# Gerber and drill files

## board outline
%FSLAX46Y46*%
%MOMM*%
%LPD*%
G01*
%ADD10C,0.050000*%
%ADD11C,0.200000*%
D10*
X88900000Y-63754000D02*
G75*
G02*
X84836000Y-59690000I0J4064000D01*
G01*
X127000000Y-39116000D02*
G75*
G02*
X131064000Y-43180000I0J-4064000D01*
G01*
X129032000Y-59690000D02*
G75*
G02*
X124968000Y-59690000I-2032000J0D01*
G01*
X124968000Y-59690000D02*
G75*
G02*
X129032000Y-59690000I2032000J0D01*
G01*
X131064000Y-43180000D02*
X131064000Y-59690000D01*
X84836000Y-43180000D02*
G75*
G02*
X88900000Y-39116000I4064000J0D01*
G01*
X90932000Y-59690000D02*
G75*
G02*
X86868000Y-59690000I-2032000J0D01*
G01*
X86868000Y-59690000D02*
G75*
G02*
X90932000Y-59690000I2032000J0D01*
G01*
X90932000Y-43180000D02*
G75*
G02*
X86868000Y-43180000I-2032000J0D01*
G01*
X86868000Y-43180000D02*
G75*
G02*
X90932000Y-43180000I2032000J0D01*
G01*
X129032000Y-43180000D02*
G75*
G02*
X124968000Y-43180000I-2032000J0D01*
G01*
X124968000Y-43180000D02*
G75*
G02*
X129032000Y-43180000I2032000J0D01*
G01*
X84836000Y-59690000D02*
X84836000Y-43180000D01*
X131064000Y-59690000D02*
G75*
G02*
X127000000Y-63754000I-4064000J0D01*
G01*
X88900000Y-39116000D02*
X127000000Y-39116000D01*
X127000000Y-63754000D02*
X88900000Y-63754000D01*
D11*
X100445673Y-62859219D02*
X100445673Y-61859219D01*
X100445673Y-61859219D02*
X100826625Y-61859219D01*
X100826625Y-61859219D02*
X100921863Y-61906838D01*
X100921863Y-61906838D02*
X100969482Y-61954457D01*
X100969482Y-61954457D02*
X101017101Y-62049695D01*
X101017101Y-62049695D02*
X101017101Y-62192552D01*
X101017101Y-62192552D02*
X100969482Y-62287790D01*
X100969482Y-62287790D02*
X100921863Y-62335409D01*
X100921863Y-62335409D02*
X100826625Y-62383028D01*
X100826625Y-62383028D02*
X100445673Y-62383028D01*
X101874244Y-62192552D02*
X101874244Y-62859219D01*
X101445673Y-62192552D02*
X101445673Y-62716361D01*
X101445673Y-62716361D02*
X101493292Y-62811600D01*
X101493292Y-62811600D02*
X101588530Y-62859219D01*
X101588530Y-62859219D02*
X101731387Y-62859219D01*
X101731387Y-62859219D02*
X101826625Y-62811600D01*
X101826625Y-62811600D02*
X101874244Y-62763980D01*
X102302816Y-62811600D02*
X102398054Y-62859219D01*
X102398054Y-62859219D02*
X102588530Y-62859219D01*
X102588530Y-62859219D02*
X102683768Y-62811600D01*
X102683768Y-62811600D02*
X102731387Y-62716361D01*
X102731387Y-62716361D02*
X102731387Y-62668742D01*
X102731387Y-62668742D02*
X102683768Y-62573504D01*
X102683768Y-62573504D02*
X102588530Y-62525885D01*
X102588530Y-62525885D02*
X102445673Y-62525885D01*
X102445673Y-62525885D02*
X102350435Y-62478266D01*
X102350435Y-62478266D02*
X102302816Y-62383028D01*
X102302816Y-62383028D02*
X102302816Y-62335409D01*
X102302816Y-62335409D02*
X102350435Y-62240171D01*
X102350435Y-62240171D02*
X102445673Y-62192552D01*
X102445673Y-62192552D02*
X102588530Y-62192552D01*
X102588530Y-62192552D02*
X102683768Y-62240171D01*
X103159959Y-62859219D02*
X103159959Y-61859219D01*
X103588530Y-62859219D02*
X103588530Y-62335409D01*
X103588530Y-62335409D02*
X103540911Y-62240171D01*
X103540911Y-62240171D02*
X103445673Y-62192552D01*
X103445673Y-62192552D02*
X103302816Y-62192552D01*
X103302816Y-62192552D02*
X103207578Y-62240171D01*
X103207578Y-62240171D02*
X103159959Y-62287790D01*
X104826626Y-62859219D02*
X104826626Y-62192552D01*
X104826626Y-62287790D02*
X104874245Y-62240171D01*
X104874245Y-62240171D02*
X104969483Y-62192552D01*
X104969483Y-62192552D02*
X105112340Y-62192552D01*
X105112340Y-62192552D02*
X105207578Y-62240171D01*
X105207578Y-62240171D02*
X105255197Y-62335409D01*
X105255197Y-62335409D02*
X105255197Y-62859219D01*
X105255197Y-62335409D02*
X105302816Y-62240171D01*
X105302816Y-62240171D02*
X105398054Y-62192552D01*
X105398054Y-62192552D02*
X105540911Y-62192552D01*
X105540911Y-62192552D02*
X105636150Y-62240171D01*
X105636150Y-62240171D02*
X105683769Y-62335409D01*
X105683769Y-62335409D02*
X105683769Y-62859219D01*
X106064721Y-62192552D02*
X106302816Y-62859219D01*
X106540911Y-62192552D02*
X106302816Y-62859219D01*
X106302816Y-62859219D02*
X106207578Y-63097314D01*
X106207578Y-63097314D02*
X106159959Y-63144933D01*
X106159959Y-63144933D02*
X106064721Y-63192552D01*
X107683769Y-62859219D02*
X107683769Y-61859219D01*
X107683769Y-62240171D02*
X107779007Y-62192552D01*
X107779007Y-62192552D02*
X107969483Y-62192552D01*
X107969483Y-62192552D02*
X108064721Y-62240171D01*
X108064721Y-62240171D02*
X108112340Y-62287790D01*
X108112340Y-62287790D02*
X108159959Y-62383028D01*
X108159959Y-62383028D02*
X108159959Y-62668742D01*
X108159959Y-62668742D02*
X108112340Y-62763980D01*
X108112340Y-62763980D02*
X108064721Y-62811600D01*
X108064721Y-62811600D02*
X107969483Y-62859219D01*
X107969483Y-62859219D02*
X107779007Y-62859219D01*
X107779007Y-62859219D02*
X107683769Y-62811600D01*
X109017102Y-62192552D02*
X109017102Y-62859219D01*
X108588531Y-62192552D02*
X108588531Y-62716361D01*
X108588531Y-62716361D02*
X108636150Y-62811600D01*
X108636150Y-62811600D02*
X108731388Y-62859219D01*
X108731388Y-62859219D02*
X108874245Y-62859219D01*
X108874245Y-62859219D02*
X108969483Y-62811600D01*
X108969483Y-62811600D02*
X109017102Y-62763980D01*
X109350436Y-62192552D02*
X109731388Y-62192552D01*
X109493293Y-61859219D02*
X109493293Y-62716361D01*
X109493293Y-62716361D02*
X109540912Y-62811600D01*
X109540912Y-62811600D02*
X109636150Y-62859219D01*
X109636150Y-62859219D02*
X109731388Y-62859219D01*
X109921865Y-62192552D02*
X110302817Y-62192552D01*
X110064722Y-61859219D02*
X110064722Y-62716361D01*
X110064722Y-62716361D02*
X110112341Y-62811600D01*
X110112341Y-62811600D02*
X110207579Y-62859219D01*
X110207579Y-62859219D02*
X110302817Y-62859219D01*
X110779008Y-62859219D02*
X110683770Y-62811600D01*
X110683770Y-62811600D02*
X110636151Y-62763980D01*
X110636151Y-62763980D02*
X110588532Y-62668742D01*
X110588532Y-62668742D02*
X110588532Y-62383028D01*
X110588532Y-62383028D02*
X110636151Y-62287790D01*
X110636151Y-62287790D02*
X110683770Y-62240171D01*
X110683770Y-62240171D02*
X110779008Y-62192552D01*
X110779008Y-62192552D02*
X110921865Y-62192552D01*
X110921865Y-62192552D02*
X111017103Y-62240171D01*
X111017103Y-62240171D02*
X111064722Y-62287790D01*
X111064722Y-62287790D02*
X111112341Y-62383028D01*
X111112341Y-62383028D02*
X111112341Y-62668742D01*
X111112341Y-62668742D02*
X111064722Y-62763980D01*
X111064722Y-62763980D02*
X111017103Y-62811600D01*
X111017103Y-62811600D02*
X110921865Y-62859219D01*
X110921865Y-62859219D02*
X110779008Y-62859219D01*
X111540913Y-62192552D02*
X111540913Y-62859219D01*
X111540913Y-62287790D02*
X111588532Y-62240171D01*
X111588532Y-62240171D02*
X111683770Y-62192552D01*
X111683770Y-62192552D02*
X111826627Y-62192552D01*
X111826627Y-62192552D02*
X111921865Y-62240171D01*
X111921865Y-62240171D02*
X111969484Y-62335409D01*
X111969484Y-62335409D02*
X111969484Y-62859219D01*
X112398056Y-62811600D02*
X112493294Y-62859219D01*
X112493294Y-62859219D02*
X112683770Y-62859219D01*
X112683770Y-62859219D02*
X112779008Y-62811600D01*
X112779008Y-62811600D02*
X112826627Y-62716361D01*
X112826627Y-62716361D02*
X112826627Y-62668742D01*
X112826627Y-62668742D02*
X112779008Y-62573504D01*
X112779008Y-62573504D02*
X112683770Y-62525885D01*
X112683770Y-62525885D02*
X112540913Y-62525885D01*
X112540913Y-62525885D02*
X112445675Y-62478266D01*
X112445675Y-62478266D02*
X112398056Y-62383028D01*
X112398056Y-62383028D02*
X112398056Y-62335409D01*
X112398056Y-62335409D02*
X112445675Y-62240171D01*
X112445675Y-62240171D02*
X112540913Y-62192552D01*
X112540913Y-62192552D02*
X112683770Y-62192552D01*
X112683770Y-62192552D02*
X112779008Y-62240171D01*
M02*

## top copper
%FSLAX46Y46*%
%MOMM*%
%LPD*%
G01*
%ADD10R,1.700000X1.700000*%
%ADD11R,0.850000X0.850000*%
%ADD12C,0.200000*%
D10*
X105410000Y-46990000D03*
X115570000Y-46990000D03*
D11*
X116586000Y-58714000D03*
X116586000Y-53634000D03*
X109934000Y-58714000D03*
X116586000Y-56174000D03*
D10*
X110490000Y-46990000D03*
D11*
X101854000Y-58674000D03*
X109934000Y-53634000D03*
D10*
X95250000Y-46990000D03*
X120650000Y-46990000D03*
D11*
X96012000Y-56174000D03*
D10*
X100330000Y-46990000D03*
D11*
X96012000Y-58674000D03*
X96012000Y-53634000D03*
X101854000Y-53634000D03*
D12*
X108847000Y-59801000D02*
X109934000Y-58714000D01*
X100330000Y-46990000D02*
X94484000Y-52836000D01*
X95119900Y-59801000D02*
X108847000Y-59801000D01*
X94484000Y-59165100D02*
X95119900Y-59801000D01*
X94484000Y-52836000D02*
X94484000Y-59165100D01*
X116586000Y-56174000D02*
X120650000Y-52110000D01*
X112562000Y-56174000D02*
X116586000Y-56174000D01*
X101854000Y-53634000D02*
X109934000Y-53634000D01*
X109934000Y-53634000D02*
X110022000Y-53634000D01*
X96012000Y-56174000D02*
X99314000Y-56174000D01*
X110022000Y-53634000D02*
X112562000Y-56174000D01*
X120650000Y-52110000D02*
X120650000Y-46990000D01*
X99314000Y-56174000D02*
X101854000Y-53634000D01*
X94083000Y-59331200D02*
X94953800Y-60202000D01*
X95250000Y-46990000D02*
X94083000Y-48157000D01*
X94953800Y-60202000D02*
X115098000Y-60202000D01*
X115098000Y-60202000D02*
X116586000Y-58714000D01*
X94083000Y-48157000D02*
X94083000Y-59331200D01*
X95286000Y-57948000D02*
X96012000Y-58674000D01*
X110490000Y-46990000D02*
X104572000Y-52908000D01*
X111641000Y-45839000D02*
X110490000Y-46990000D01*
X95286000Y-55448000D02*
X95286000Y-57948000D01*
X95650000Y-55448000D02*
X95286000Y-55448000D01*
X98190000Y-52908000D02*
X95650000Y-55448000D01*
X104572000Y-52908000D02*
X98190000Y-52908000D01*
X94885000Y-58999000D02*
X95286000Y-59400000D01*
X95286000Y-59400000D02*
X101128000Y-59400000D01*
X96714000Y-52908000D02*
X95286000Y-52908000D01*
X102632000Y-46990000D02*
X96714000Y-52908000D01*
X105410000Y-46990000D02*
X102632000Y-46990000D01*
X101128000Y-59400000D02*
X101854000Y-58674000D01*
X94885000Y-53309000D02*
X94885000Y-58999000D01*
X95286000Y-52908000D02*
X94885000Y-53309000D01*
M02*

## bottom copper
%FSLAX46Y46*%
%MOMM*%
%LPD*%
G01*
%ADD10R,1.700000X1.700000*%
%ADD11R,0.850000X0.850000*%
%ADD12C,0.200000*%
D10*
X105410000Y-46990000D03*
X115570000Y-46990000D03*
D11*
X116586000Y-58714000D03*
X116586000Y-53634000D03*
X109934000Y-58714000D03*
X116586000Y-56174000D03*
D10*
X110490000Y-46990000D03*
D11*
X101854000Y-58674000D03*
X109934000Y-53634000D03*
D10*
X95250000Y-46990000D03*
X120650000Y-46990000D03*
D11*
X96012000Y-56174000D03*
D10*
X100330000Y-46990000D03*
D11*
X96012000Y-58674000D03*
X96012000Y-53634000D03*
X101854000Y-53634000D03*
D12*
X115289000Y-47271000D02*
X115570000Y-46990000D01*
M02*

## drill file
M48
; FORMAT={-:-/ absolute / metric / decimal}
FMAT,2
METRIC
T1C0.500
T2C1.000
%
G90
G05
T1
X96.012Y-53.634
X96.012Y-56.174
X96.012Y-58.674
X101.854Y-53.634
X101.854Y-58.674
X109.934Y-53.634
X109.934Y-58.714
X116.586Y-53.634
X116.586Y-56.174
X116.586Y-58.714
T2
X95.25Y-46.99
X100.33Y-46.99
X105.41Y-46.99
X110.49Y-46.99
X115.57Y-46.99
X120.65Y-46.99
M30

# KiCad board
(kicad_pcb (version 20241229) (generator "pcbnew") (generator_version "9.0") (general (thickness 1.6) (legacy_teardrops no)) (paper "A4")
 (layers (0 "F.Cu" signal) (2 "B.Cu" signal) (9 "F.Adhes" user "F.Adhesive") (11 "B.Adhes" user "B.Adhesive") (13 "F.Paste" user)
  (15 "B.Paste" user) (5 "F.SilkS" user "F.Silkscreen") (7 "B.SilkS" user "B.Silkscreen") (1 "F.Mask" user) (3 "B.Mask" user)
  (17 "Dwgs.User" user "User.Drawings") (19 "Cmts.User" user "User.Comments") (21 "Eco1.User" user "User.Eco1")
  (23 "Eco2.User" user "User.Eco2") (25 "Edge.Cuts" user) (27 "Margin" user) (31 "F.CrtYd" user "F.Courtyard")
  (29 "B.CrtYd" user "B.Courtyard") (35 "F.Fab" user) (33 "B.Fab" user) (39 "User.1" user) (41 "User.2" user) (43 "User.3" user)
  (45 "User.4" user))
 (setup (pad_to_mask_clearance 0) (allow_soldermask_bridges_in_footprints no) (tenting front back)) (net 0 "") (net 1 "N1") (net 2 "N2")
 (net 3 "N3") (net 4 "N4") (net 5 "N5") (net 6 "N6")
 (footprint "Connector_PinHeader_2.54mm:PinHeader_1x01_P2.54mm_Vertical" (layer "F.Cu") (at 105.41 46.99)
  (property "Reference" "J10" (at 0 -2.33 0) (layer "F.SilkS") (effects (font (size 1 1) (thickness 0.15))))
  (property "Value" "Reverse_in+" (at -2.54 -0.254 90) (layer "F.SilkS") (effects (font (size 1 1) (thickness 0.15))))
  (pad "1" thru_hole rect (at 0 0) (size 1.7 1.7) (drill 1) (layers "*.Cu" "*.Mask") (remove_unused_layers no) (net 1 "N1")))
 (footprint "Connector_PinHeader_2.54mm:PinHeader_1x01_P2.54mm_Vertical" (layer "F.Cu") (at 115.57 46.99)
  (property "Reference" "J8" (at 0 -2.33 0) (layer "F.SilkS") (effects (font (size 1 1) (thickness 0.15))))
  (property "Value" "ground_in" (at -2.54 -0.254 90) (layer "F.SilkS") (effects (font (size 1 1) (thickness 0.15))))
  (pad "1" thru_hole rect (at 0 0) (size 1.7 1.7) (drill 1) (layers "*.Cu" "*.Mask") (remove_unused_layers no) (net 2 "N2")))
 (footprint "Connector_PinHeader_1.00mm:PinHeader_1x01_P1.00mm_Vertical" (layer "F.Cu") (at 116.586 58.714)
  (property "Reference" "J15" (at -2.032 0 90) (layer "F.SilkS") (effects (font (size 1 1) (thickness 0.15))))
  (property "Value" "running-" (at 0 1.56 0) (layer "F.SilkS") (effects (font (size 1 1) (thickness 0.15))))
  (pad "1" thru_hole rect (at 0 0) (size 0.85 0.85) (drill 0.5) (layers "*.Cu" "*.Mask") (remove_unused_layers no) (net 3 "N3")))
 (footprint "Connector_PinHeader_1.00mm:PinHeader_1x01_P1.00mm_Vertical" (layer "F.Cu") (at 116.586 53.634)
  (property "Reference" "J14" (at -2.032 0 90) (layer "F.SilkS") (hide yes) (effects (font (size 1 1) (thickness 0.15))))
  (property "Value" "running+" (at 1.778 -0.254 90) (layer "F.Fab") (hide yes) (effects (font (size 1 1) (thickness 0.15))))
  (pad "1" thru_hole rect (at 0 0) (size 0.85 0.85) (drill 0.5) (layers "*.Cu" "*.Mask") (remove_unused_layers no)))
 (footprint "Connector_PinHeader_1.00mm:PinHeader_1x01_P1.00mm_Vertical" (layer "F.Cu") (at 109.934 58.714)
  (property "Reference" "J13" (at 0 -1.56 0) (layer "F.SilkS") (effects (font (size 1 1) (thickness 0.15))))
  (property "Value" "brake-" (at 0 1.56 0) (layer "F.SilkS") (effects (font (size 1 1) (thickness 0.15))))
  (pad "1" thru_hole rect (at 0 0) (size 0.85 0.85) (drill 0.5) (layers "*.Cu" "*.Mask") (remove_unused_layers no) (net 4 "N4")))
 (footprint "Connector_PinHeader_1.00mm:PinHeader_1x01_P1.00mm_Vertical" (layer "F.Cu") (at 116.586 56.174)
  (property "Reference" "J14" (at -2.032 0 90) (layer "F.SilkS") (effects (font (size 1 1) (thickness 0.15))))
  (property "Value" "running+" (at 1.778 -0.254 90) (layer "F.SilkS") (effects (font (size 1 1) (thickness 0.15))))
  (pad "1" thru_hole rect (at 0 0) (size 0.85 0.85) (drill 0.5) (layers "*.Cu" "*.Mask") (remove_unused_layers no) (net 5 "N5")))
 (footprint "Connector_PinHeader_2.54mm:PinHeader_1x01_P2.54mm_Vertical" (layer "F.Cu") (at 110.49 46.99)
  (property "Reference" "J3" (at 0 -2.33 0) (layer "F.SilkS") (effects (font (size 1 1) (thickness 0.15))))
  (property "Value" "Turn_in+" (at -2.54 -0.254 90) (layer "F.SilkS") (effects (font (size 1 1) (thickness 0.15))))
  (pad "1" thru_hole rect (at 0 0) (size 1.7 1.7) (drill 1) (layers "*.Cu" "*.Mask") (remove_unused_layers no) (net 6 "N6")))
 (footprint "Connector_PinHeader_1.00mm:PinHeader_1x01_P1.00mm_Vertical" (layer "F.Cu") (at 101.854 58.674)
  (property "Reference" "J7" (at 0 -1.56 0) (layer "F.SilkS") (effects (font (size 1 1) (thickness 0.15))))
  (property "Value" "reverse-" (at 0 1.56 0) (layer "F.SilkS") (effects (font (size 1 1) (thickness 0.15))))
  (pad "1" thru_hole rect (at 0 0) (size 0.85 0.85) (drill 0.5) (layers "*.Cu" "*.Mask") (remove_unused_layers no) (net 1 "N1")))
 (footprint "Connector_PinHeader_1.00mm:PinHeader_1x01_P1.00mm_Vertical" (layer "F.Cu") (at 109.934 53.634)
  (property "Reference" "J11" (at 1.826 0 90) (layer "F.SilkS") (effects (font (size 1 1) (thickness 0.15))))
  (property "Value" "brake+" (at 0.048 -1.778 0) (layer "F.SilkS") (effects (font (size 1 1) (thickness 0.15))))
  (pad "1" thru_hole rect (at 0 0) (size 0.85 0.85) (drill 0.5) (layers "*.Cu" "*.Mask") (remove_unused_layers no) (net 5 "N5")))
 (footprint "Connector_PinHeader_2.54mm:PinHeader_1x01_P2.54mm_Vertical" (layer "F.Cu") (at 95.25 46.99)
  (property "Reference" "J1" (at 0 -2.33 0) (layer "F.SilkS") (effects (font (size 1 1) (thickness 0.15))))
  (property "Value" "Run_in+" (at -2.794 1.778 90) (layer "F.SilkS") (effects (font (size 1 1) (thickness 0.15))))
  (pad "1" thru_hole rect (at 0 0) (size 1.7 1.7) (drill 1) (layers "*.Cu" "*.Mask") (remove_unused_layers no) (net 3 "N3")))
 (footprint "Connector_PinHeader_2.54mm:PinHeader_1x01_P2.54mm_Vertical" (layer "F.Cu") (at 120.65 46.99)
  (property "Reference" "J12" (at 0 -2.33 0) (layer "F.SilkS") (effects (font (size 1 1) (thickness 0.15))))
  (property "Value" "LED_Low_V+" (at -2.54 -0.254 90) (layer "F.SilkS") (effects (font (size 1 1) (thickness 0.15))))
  (pad "1" thru_hole rect (at 0 0) (size 1.7 1.7) (drill 1) (layers "*.Cu" "*.Mask") (remove_unused_layers no) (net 5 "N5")))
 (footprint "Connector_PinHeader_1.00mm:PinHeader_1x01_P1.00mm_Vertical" (layer "F.Cu") (at 96.012 56.174)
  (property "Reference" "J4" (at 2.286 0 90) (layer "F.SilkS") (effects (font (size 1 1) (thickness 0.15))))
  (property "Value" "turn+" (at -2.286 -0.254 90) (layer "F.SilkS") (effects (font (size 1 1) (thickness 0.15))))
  (pad "1" thru_hole rect (at 0 0) (size 0.85 0.85) (drill 0.5) (layers "*.Cu" "*.Mask") (remove_unused_layers no) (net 5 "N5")))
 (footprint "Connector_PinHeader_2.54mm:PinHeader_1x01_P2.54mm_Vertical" (layer "F.Cu") (at 100.33 46.99)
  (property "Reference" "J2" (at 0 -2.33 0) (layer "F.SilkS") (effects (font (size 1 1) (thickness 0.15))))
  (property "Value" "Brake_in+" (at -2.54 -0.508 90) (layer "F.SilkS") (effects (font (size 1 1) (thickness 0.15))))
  (pad "1" thru_hole rect (at 0 0) (size 1.7 1.7) (drill 1) (layers "*.Cu" "*.Mask") (remove_unused_layers no) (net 4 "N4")))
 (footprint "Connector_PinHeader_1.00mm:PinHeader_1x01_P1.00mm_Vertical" (layer "F.Cu") (at 96.012 58.674)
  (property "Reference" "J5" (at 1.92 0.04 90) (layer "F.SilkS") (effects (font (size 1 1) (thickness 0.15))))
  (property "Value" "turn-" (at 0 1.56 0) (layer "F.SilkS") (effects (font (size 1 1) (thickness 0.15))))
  (pad "1" thru_hole rect (at 0 0) (size 0.85 0.85) (drill 0.5) (layers "*.Cu" "*.Mask") (remove_unused_layers no) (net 6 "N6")))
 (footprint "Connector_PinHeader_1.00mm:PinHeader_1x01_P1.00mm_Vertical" (layer "F.Cu") (at 96.012 53.634)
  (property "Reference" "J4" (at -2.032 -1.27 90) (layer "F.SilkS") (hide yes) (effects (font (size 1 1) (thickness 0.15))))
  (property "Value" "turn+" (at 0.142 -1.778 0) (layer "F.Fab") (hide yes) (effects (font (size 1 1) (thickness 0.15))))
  (pad "1" thru_hole rect (at 0 0) (size 0.85 0.85) (drill 0.5) (layers "*.Cu" "*.Mask") (remove_unused_layers no)))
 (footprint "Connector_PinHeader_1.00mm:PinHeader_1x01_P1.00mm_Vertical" (layer "F.Cu") (at 101.854 53.634)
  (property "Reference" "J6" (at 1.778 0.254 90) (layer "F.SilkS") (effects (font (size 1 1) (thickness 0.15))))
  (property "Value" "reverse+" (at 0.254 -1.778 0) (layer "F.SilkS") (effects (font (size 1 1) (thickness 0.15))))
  (pad "1" thru_hole rect (at 0 0) (size 0.85 0.85) (drill 0.5) (layers "*.Cu" "*.Mask") (remove_unused_layers no) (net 5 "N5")))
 (gr_arc (start 88.9 63.754) (mid 86.026318 62.563682) (end 84.836 59.69) (stroke (width 0.05) (type default)) (layer "Edge.Cuts"))
 (gr_arc (start 127 39.116) (mid 129.873682 40.306318) (end 131.064 43.18) (stroke (width 0.05) (type default)) (layer "Edge.Cuts"))
 (gr_circle (center 127 59.69) (end 124.968 59.69) (stroke (width 0.05) (type default)) (fill no) (layer "Edge.Cuts"))
 (gr_line (start 131.064 43.18) (end 131.064 59.69) (stroke (width 0.05) (type default)) (layer "Edge.Cuts"))
 (gr_arc (start 84.836 43.18) (mid 86.026318 40.306318) (end 88.9 39.116) (stroke (width 0.05) (type default)) (layer "Edge.Cuts"))
 (gr_circle (center 88.9 59.69) (end 86.868 59.69) (stroke (width 0.05) (type default)) (fill no) (layer "Edge.Cuts"))
 (gr_circle (center 88.9 43.18) (end 90.932 43.18) (stroke (width 0.05) (type default)) (fill no) (layer "Edge.Cuts"))
 (gr_circle (center 127 43.18) (end 129.032 43.18) (stroke (width 0.05) (type default)) (fill no) (layer "Edge.Cuts"))
 (gr_line (start 84.836 59.69) (end 84.836 43.18) (stroke (width 0.05) (type default)) (layer "Edge.Cuts"))
 (gr_arc (start 131.064 59.69) (mid 129.873682 62.563682) (end 127 63.754) (stroke (width 0.05) (type default)) (layer "Edge.Cuts"))
 (gr_line (start 88.9 39.116) (end 127 39.116) (stroke (width 0.05) (type default)) (layer "Edge.Cuts"))
 (gr_line (start 127 63.754) (end 88.9 63.754) (stroke (width 0.05) (type default)) (layer "Edge.Cuts"))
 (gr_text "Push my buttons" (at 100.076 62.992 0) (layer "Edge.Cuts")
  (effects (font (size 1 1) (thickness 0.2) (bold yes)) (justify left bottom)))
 (segment (start 108.847 59.801) (end 109.934 58.714) (width 0.2) (layer "F.Cu") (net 4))
 (segment (start 100.33 46.99) (end 94.484 52.836) (width 0.2) (layer "F.Cu") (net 4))
 (segment (start 95.1199 59.801) (end 108.847 59.801) (width 0.2) (layer "F.Cu") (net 4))
 (segment (start 94.484 59.1651) (end 95.1199 59.801) (width 0.2) (layer "F.Cu") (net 4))
 (segment (start 94.484 52.836) (end 94.484 59.1651) (width 0.2) (layer "F.Cu") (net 4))
 (segment (start 116.586 56.174) (end 120.65 52.11) (width 0.2) (layer "F.Cu") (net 5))
 (segment (start 112.562 56.174) (end 116.586 56.174) (width 0.2) (layer "F.Cu") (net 5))
 (segment (start 101.854 53.634) (end 109.934 53.634) (width 0.2) (layer "F.Cu") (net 5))
 (segment (start 109.934 53.634) (end 110.022 53.634) (width 0.2) (layer "F.Cu") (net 5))
 (segment (start 96.012 56.174) (end 99.314 56.174) (width 0.2) (layer "F.Cu") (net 5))
 (segment (start 110.022 53.634) (end 112.562 56.174) (width 0.2) (layer "F.Cu") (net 5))
 (segment (start 120.65 52.11) (end 120.65 46.99) (width 0.2) (layer "F.Cu") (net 5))
 (segment (start 99.314 56.174) (end 101.854 53.634) (width 0.2) (layer "F.Cu") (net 5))
 (segment (start 94.083 59.3312) (end 94.9538 60.202) (width 0.2) (layer "F.Cu") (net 3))
 (segment (start 95.25 46.99) (end 94.083 48.157) (width 0.2) (layer "F.Cu") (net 3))
 (segment (start 94.9538 60.202) (end 115.098 60.202) (width 0.2) (layer "F.Cu") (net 3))
 (segment (start 115.098 60.202) (end 116.586 58.714) (width 0.2) (layer "F.Cu") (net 3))
 (segment (start 94.083 48.157) (end 94.083 59.3312) (width 0.2) (layer "F.Cu") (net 3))
 (segment (start 115.289 47.271) (end 115.57 46.99) (width 0.2) (layer "B.Cu") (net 2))
 (segment (start 95.286 57.948) (end 96.012 58.674) (width 0.2) (layer "F.Cu") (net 6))
 (segment (start 110.49 46.99) (end 104.572 52.908) (width 0.2) (layer "F.Cu") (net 6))
 (segment (start 111.641 45.839) (end 110.49 46.99) (width 0.2) (layer "F.Cu") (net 6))
 (segment (start 95.286 55.448) (end 95.286 57.948) (width 0.2) (layer "F.Cu") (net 6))
 (segment (start 95.65 55.448) (end 95.286 55.448) (width 0.2) (layer "F.Cu") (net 6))
 (segment (start 98.19 52.908) (end 95.65 55.448) (width 0.2) (layer "F.Cu") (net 6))
 (segment (start 104.572 52.908) (end 98.19 52.908) (width 0.2) (layer "F.Cu") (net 6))
 (segment (start 94.885 58.999) (end 95.286 59.4) (width 0.2) (layer "F.Cu") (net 1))
 (segment (start 95.286 59.4) (end 101.128 59.4) (width 0.2) (layer "F.Cu") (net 1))
 (segment (start 96.714 52.908) (end 95.286 52.908) (width 0.2) (layer "F.Cu") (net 1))
 (segment (start 102.632 46.99) (end 96.714 52.908) (width 0.2) (layer "F.Cu") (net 1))
 (segment (start 105.41 46.99) (end 102.632 46.99) (width 0.2) (layer "F.Cu") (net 1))
 (segment (start 101.128 59.4) (end 101.854 58.674) (width 0.2) (layer "F.Cu") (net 1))
 (segment (start 94.885 53.309) (end 94.885 58.999) (width 0.2) (layer "F.Cu") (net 1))
 (segment (start 95.286 52.908) (end 94.885 53.309) (width 0.2) (layer "F.Cu") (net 1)))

